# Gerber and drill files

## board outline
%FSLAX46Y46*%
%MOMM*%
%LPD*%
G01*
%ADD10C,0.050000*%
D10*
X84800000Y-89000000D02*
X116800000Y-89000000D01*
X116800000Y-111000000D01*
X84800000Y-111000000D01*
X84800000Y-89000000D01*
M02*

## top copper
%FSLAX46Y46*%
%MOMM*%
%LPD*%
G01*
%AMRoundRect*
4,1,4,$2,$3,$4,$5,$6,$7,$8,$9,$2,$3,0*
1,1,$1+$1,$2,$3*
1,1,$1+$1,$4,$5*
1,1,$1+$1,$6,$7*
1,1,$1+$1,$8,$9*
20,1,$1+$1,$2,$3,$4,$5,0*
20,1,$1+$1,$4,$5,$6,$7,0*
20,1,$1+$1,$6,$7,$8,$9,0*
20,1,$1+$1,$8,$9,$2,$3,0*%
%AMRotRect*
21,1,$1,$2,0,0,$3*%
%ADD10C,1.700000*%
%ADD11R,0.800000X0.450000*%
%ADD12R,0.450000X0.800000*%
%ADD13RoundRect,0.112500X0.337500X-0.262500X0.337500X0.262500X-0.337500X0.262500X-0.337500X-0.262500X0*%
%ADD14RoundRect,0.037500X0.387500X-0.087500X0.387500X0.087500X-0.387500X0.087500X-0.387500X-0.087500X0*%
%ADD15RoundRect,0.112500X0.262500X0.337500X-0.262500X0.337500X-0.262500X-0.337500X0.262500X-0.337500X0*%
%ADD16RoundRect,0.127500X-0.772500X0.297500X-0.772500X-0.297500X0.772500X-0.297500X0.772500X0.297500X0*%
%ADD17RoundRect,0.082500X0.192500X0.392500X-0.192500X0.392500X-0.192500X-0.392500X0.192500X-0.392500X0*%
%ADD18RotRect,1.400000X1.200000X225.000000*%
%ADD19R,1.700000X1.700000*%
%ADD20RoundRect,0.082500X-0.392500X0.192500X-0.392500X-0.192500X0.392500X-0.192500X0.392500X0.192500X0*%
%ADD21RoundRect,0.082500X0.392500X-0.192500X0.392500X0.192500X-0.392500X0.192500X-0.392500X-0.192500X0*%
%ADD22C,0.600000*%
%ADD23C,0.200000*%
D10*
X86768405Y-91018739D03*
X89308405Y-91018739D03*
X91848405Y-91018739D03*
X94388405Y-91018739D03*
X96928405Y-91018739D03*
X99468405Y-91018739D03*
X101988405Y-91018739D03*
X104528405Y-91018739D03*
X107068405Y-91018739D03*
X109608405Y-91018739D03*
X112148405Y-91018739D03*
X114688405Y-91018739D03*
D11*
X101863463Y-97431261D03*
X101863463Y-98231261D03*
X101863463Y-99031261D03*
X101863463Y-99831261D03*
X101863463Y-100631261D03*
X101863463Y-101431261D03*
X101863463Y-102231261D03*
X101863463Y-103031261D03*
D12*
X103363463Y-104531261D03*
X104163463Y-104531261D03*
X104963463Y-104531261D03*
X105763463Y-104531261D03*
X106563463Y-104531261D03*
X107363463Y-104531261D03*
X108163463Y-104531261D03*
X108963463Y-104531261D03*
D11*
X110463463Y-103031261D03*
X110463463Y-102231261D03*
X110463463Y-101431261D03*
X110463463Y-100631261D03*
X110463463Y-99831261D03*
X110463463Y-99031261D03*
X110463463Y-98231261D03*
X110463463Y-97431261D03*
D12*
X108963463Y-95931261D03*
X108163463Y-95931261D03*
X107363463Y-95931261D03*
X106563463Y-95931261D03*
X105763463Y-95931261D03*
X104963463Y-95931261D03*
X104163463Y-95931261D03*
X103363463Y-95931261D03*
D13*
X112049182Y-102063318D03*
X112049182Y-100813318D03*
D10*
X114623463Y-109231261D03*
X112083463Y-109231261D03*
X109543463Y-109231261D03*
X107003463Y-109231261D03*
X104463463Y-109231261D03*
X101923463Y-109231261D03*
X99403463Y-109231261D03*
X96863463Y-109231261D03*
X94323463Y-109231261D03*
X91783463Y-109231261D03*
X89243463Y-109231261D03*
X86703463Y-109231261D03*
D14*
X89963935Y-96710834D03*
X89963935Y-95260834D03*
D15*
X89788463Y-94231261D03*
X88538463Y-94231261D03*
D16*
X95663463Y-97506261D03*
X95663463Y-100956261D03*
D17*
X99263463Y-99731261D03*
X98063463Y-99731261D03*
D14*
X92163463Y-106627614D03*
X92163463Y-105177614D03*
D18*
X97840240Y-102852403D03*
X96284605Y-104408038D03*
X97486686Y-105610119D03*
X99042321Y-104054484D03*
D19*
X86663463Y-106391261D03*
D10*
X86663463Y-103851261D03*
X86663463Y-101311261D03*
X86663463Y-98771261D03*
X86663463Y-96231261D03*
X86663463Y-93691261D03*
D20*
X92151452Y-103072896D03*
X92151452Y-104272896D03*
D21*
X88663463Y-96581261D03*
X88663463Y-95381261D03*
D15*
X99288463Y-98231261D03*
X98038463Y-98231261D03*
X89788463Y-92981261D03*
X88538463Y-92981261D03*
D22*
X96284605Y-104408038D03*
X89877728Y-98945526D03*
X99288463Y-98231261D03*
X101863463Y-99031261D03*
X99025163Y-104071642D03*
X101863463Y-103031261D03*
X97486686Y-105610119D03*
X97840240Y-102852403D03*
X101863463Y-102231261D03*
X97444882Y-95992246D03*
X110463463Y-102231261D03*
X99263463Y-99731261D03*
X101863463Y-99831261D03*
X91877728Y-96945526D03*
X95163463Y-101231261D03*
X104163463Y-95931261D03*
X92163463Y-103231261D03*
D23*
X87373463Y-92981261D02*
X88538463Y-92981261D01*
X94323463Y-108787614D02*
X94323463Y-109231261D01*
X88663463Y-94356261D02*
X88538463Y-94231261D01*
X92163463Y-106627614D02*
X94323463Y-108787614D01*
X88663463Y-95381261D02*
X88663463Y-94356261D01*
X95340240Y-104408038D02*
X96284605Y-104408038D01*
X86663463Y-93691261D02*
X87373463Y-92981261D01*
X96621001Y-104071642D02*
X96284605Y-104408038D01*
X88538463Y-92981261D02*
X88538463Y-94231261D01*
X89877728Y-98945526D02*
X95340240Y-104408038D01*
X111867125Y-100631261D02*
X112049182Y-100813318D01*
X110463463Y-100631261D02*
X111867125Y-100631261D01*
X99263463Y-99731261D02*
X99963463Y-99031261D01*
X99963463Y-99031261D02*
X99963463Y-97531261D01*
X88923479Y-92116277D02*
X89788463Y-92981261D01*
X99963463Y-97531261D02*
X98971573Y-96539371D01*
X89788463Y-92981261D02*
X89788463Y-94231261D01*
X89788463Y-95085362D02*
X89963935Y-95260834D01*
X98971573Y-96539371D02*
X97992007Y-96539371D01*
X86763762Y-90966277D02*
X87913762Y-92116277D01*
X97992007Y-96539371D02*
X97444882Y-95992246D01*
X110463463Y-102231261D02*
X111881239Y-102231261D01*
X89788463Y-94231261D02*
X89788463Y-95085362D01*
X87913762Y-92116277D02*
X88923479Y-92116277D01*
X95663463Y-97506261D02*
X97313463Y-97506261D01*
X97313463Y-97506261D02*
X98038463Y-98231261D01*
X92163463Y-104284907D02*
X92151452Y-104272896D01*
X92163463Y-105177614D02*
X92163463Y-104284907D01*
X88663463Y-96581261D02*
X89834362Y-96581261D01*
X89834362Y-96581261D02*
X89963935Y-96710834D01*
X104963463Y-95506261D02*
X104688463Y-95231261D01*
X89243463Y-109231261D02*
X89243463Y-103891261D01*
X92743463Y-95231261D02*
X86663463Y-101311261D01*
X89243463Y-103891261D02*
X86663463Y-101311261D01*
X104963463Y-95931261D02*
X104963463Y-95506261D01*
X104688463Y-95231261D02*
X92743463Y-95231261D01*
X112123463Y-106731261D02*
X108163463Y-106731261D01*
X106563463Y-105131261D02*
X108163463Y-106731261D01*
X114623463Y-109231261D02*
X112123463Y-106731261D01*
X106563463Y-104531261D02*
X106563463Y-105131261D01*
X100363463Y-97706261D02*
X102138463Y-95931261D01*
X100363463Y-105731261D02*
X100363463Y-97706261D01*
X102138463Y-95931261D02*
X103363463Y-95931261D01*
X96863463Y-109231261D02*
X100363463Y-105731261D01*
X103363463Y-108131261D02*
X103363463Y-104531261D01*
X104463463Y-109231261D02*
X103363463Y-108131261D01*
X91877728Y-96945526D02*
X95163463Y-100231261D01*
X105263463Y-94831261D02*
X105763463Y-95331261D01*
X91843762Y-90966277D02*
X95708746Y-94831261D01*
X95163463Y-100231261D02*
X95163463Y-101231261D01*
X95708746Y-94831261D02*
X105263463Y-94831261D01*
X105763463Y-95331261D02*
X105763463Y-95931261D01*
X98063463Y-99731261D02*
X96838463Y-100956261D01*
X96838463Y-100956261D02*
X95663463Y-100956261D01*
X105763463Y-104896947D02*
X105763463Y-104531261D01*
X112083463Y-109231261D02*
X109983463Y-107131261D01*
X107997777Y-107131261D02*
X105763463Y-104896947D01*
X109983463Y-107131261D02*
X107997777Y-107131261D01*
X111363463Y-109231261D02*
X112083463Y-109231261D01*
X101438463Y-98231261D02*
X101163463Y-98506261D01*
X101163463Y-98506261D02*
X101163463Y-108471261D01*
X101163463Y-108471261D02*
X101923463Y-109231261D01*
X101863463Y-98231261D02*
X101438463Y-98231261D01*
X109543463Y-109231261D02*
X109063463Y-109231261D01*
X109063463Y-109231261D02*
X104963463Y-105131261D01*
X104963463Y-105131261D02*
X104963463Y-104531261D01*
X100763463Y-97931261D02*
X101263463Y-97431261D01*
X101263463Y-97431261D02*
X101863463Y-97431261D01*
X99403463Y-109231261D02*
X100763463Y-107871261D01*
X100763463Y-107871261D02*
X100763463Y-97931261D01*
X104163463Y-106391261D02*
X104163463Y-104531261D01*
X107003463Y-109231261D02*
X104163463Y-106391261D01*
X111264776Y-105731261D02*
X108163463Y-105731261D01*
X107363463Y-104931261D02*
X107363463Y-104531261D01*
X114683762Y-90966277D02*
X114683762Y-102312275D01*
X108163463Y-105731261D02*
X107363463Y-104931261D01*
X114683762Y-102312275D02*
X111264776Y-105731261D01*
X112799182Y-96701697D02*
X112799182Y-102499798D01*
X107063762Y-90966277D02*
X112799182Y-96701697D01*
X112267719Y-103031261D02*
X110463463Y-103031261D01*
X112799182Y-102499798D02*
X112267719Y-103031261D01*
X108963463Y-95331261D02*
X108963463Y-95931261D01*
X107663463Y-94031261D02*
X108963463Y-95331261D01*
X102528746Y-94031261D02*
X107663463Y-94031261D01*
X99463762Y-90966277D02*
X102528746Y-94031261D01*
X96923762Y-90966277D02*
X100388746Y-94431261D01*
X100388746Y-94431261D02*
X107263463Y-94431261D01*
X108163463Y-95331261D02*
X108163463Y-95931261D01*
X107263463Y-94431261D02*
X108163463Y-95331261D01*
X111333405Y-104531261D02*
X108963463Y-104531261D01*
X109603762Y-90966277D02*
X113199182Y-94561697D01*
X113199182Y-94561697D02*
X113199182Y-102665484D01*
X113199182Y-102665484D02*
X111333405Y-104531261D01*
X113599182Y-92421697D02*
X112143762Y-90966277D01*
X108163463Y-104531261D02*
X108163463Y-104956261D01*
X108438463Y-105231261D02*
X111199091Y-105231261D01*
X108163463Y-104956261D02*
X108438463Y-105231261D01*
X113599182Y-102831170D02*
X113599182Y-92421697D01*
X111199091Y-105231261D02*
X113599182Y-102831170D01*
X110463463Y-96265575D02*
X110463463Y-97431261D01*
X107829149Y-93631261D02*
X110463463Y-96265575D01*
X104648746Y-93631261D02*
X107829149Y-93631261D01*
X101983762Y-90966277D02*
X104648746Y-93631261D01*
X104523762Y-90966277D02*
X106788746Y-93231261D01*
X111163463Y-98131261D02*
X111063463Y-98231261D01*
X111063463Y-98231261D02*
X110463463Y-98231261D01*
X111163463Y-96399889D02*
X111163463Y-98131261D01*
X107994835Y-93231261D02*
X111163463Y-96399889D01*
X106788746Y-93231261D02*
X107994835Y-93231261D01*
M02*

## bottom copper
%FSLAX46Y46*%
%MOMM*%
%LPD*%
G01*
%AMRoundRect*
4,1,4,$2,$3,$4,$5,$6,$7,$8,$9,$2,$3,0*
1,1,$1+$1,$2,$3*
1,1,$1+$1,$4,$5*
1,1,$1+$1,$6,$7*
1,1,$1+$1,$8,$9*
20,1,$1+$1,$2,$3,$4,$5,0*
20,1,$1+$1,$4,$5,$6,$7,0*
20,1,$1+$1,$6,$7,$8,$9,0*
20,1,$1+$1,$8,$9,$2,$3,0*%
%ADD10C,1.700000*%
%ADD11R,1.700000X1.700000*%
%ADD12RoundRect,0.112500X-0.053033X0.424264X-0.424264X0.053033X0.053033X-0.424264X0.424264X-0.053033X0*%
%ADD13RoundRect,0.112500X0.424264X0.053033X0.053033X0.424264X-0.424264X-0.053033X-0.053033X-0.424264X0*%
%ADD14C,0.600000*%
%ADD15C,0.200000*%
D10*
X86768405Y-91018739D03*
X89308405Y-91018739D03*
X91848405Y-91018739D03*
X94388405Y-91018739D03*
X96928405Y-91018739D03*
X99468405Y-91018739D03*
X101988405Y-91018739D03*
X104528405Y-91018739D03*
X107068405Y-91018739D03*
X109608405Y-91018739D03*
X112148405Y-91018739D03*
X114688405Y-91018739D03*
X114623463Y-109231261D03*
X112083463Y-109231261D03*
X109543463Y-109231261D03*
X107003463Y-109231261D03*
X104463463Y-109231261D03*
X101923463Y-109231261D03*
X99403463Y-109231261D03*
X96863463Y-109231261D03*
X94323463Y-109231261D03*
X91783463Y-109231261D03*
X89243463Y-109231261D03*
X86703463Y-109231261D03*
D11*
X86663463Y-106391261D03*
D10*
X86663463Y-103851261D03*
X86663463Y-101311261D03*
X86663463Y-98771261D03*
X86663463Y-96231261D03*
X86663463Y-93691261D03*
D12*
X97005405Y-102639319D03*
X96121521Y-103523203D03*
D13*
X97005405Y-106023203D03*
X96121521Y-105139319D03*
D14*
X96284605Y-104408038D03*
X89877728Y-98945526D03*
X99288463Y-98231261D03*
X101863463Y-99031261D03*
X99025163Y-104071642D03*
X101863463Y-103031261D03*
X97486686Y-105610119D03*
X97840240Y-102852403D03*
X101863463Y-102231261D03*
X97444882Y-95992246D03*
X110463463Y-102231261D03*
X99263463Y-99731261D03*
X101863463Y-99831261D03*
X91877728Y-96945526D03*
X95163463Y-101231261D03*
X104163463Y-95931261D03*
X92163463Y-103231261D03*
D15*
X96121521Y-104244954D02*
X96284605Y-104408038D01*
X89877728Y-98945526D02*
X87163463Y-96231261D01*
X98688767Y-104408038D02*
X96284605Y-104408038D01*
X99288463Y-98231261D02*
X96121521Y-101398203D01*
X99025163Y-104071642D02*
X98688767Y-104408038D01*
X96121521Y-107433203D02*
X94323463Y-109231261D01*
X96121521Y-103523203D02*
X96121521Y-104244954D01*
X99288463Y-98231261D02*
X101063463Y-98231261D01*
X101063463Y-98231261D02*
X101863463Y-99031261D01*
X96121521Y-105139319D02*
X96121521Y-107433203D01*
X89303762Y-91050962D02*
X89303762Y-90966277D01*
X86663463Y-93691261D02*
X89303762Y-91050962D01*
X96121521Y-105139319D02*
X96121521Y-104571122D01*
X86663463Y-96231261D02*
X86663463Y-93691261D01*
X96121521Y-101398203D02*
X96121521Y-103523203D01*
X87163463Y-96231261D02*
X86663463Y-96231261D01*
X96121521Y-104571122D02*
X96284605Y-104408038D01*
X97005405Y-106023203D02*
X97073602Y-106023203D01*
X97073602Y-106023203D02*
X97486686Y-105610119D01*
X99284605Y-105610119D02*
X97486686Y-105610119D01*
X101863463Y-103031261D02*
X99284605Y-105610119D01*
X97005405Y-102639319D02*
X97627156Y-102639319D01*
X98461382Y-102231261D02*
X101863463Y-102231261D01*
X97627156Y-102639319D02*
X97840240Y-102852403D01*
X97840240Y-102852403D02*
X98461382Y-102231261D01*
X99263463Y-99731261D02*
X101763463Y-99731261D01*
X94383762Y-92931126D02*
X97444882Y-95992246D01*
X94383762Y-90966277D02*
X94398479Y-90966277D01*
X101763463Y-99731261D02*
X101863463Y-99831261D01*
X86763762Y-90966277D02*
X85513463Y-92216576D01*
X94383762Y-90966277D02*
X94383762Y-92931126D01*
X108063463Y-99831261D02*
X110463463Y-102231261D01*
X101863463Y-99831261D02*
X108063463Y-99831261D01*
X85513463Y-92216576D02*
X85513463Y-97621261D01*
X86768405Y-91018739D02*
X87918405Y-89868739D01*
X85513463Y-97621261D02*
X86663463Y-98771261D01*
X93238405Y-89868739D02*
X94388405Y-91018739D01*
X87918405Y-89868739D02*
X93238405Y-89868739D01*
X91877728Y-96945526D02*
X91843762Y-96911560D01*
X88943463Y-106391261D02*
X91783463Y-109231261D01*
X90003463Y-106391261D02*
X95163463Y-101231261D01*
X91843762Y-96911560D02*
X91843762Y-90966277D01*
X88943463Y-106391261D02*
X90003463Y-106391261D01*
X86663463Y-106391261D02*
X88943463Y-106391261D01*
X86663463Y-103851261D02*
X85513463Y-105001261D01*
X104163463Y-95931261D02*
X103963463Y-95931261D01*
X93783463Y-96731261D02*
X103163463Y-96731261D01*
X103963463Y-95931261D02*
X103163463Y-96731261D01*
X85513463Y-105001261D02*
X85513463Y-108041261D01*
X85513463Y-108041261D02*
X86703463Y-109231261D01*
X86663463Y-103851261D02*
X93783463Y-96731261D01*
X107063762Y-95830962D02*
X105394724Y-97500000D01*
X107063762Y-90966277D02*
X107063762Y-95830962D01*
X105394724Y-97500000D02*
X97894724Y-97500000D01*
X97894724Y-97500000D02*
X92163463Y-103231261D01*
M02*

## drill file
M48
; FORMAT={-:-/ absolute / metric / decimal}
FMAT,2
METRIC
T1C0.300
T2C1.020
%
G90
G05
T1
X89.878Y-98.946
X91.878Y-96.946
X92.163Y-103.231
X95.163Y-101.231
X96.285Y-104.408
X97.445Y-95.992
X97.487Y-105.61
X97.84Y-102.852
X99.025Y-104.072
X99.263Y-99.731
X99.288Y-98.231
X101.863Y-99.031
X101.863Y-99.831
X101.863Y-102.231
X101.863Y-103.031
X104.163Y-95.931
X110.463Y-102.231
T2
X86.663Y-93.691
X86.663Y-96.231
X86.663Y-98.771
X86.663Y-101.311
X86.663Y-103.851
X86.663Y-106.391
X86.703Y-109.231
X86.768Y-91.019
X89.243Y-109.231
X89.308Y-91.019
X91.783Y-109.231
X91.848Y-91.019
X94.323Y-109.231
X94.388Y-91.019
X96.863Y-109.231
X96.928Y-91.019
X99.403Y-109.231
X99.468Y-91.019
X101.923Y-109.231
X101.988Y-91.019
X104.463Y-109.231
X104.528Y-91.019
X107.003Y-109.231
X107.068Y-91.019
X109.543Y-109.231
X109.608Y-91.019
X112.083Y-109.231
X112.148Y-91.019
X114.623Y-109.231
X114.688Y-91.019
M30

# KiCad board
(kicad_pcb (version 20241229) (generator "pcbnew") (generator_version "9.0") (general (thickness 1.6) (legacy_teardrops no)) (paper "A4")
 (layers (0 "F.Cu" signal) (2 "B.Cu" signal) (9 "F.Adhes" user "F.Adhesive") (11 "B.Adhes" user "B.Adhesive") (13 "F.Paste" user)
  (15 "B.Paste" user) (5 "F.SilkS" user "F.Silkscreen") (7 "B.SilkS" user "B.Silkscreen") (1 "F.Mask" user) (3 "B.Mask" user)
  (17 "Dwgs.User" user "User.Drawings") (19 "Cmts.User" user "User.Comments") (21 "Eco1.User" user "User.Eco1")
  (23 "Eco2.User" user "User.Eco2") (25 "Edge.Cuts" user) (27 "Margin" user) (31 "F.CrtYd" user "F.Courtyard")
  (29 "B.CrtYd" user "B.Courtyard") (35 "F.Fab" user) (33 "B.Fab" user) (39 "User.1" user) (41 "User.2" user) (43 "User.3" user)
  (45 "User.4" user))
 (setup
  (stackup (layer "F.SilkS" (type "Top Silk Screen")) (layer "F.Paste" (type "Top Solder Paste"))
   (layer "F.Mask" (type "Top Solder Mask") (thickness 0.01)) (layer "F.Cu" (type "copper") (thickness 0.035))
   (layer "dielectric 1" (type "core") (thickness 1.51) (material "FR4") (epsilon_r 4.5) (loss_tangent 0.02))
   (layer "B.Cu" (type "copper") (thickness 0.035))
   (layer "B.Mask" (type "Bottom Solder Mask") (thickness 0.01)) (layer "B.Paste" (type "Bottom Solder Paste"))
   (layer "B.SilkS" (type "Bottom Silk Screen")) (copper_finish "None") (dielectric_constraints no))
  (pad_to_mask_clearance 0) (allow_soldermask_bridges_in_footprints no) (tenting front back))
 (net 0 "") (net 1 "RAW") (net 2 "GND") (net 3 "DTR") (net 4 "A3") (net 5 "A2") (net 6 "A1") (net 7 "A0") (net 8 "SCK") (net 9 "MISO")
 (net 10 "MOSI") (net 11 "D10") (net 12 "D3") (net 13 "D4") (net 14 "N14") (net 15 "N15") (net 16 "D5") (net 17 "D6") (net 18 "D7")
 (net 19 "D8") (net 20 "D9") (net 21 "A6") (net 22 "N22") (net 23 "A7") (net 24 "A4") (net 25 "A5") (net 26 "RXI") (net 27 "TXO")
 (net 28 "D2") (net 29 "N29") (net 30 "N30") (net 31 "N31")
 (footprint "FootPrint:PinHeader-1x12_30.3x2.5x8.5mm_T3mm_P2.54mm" (layer "F.Cu") (at 100.728405 91.018739)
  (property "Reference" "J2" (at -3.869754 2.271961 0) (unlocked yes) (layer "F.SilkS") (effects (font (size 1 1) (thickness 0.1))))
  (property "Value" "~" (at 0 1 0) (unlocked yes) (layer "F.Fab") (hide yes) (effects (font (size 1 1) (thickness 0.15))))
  (pad "1" thru_hole circle (at -13.96 0) (size 1.7 1.7) (drill 1.02) (layers "*.Cu" "*.Mask") (remove_unused_layers no) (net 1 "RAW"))
  (pad "2" thru_hole circle (at -11.42 0) (size 1.7 1.7) (drill 1.02) (layers "*.Cu" "*.Mask") (remove_unused_layers no) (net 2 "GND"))
  (pad "3" thru_hole circle (at -8.88 0) (size 1.7 1.7) (drill 1.02) (layers "*.Cu" "*.Mask") (remove_unused_layers no) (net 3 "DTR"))
  (pad "4" thru_hole circle (at -6.34 0) (size 1.7 1.7) (drill 1.02) (layers "*.Cu" "*.Mask") (remove_unused_layers no) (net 1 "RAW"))
  (pad "5" thru_hole circle (at -3.8 0) (size 1.7 1.7) (drill 1.02) (layers "*.Cu" "*.Mask") (remove_unused_layers no) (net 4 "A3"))
  (pad "6" thru_hole circle (at -1.26 0) (size 1.7 1.7) (drill 1.02) (layers "*.Cu" "*.Mask") (remove_unused_layers no) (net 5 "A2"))
  (pad "7" thru_hole circle (at 1.26 0) (size 1.7 1.7) (drill 1.02) (layers "*.Cu" "*.Mask") (remove_unused_layers no) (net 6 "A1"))
  (pad "8" thru_hole circle (at 3.8 0) (size 1.7 1.7) (drill 1.02) (layers "*.Cu" "*.Mask") (remove_unused_layers no) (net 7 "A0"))
  (pad "9" thru_hole circle (at 6.34 0) (size 1.7 1.7) (drill 1.02) (layers "*.Cu" "*.Mask") (remove_unused_layers no) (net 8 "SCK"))
  (pad "10" thru_hole circle (at 8.88 0) (size 1.7 1.7) (drill 1.02) (layers "*.Cu" "*.Mask") (remove_unused_layers no) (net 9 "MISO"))
  (pad "11" thru_hole circle (at 11.42 0) (size 1.7 1.7) (drill 1.02) (layers "*.Cu" "*.Mask") (remove_unused_layers no) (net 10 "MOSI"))
  (pad "12" thru_hole circle (at 13.96 0) (size 1.7 1.7) (drill 1.02) (layers "*.Cu" "*.Mask") (remove_unused_layers no) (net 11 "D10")))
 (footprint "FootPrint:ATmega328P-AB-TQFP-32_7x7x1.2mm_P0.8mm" (layer "F.Cu") (at 106.163463 100.231261)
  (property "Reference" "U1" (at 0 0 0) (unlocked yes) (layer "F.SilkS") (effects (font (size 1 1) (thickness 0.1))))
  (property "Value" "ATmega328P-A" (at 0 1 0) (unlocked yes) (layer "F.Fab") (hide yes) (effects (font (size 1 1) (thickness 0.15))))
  (pad "1" smd rect (at -4.3 -2.8) (size 0.8 0.45) (layers "F.Cu" "F.Mask" "F.Paste") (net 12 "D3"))
  (pad "2" smd rect (at -4.3 -2) (size 0.8 0.45) (layers "F.Cu" "F.Mask" "F.Paste") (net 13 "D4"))
  (pad "3" smd rect (at -4.3 -1.2) (size 0.8 0.45) (layers "F.Cu" "F.Mask" "F.Paste") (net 2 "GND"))
  (pad "4" smd rect (at -4.3 -0.4) (size 0.8 0.45) (layers "F.Cu" "F.Mask" "F.Paste") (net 1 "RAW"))
  (pad "5" smd rect (at -4.3 0.4) (size 0.8 0.45) (layers "F.Cu" "F.Mask" "F.Paste"))
  (pad "6" smd rect (at -4.3 1.2) (size 0.8 0.45) (layers "F.Cu" "F.Mask" "F.Paste"))
  (pad "7" smd rect (at -4.3 2) (size 0.8 0.45) (layers "F.Cu" "F.Mask" "F.Paste") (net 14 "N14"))
  (pad "8" smd rect (at -4.3 2.8) (size 0.8 0.45) (layers "F.Cu" "F.Mask" "F.Paste") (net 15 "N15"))
  (pad "9" smd rect (at -2.8 4.3 90) (size 0.8 0.45) (layers "F.Cu" "F.Mask" "F.Paste") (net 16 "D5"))
  (pad "10" smd rect (at -2 4.3 90) (size 0.8 0.45) (layers "F.Cu" "F.Mask" "F.Paste") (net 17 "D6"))
  (pad "11" smd rect (at -1.2 4.3 90) (size 0.8 0.45) (layers "F.Cu" "F.Mask" "F.Paste") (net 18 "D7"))
  (pad "12" smd rect (at -0.4 4.3 90) (size 0.8 0.45) (layers "F.Cu" "F.Mask" "F.Paste") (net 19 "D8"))
  (pad "13" smd rect (at 0.4 4.3 90) (size 0.8 0.45) (layers "F.Cu" "F.Mask" "F.Paste") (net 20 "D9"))
  (pad "14" smd rect (at 1.2 4.3 90) (size 0.8 0.45) (layers "F.Cu" "F.Mask" "F.Paste") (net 11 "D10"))
  (pad "15" smd rect (at 2 4.3 90) (size 0.8 0.45) (layers "F.Cu" "F.Mask" "F.Paste") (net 10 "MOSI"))
  (pad "16" smd rect (at 2.8 4.3 90) (size 0.8 0.45) (layers "F.Cu" "F.Mask" "F.Paste") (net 9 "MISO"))
  (pad "17" smd rect (at 4.3 2.8) (size 0.8 0.45) (layers "F.Cu" "F.Mask" "F.Paste") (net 8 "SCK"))
  (pad "18" smd rect (at 4.3 2) (size 0.8 0.45) (layers "F.Cu" "F.Mask" "F.Paste") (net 1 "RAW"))
  (pad "19" smd rect (at 4.3 1.2) (size 0.8 0.45) (layers "F.Cu" "F.Mask" "F.Paste") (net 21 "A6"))
  (pad "20" smd rect (at 4.3 0.4) (size 0.8 0.45) (layers "F.Cu" "F.Mask" "F.Paste") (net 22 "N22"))
  (pad "21" smd rect (at 4.3 -0.4) (size 0.8 0.45) (layers "F.Cu" "F.Mask" "F.Paste"))
  (pad "22" smd rect (at 4.3 -1.2) (size 0.8 0.45) (layers "F.Cu" "F.Mask" "F.Paste") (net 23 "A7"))
  (pad "23" smd rect (at 4.3 -2) (size 0.8 0.45) (layers "F.Cu" "F.Mask" "F.Paste") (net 7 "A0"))
  (pad "24" smd rect (at 4.3 -2.8) (size 0.8 0.45) (layers "F.Cu" "F.Mask" "F.Paste") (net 6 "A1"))
  (pad "25" smd rect (at 2.8 -4.3 90) (size 0.8 0.45) (layers "F.Cu" "F.Mask" "F.Paste") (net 5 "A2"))
  (pad "26" smd rect (at 2 -4.3 90) (size 0.8 0.45) (layers "F.Cu" "F.Mask" "F.Paste") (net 4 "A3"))
  (pad "27" smd rect (at 1.2 -4.3 90) (size 0.8 0.45) (layers "F.Cu" "F.Mask" "F.Paste") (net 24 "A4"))
  (pad "28" smd rect (at 0.4 -4.3 90) (size 0.8 0.45) (layers "F.Cu" "F.Mask" "F.Paste") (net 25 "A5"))
  (pad "29" smd rect (at -0.4 -4.3 90) (size 0.8 0.45) (layers "F.Cu" "F.Mask" "F.Paste") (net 3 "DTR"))
  (pad "30" smd rect (at -1.2 -4.3 90) (size 0.8 0.45) (layers "F.Cu" "F.Mask" "F.Paste") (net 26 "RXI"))
  (pad "31" smd rect (at -2 -4.3 90) (size 0.8 0.45) (layers "F.Cu" "F.Mask" "F.Paste") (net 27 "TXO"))
  (pad "32" smd rect (at -2.8 -4.3 90) (size 0.8 0.45) (layers "F.Cu" "F.Mask" "F.Paste") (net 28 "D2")))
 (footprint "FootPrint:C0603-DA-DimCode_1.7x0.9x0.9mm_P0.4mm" (layer "F.Cu") (at 112.049182 101.438318 90)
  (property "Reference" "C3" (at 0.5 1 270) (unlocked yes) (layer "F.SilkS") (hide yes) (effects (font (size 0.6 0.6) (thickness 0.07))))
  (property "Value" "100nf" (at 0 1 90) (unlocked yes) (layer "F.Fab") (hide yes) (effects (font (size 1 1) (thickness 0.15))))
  (pad "1" smd roundrect (at -0.625 0 90) (size 0.75 0.9) (layers "F.Cu" "F.Mask" "F.Paste") (roundrect_rratio 0.15) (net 1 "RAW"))
  (pad "2" smd roundrect (at 0.625 0 90) (size 0.75 0.9) (layers "F.Cu" "F.Mask" "F.Paste") (roundrect_rratio 0.15) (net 22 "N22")))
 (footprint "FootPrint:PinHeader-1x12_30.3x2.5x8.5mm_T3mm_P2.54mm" (layer "F.Cu") (at 100.663463 109.231261 180)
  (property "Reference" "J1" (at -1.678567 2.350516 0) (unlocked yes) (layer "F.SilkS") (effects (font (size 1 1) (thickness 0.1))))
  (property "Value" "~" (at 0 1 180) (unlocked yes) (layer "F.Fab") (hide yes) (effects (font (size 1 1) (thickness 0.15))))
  (pad "1" thru_hole circle (at -13.96 0 180) (size 1.7 1.7) (drill 1.02) (layers "*.Cu" "*.Mask") (remove_unused_layers no) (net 20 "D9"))
  (pad "2" thru_hole circle (at -11.42 0 180) (size 1.7 1.7) (drill 1.02) (layers "*.Cu" "*.Mask") (remove_unused_layers no) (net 19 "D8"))
  (pad "3" thru_hole circle (at -8.88 0 180) (size 1.7 1.7) (drill 1.02) (layers "*.Cu" "*.Mask") (remove_unused_layers no) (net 18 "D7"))
  (pad "4" thru_hole circle (at -6.34 0 180) (size 1.7 1.7) (drill 1.02) (layers "*.Cu" "*.Mask") (remove_unused_layers no) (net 17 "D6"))
  (pad "5" thru_hole circle (at -3.8 0 180) (size 1.7 1.7) (drill 1.02) (layers "*.Cu" "*.Mask") (remove_unused_layers no) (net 16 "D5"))
  (pad "6" thru_hole circle (at -1.26 0 180) (size 1.7 1.7) (drill 1.02) (layers "*.Cu" "*.Mask") (remove_unused_layers no) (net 13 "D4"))
  (pad "7" thru_hole circle (at 1.26 0 180) (size 1.7 1.7) (drill 1.02) (layers "*.Cu" "*.Mask") (remove_unused_layers no) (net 12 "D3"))
  (pad "8" thru_hole circle (at 3.8 0 180) (size 1.7 1.7) (drill 1.02) (layers "*.Cu" "*.Mask") (remove_unused_layers no) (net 28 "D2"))
  (pad "9" thru_hole circle (at 6.34 0 180) (size 1.7 1.7) (drill 1.02) (layers "*.Cu" "*.Mask") (remove_unused_layers no) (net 2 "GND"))
  (pad "10" thru_hole circle (at 8.88 0 180) (size 1.7 1.7) (drill 1.02) (layers "*.Cu" "*.Mask") (remove_unused_layers no) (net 3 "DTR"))
  (pad "11" thru_hole circle (at 11.42 0 180) (size 1.7 1.7) (drill 1.02) (layers "*.Cu" "*.Mask") (remove_unused_layers no) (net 26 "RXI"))
  (pad "12" thru_hole circle (at 13.96 0 180) (size 1.7 1.7) (drill 1.02) (layers "*.Cu" "*.Mask") (remove_unused_layers no) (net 27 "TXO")))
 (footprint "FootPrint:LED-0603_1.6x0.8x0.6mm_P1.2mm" (layer "F.Cu") (at 89.963935 95.985834 90)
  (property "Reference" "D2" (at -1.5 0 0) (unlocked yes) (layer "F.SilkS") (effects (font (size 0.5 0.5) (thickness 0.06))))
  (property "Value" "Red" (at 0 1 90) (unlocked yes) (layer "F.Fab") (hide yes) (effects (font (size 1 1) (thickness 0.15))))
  (pad "1" smd roundrect (at -0.725 0 90) (size 0.25 0.85) (layers "F.Cu" "F.Mask" "F.Paste") (roundrect_rratio 0.15) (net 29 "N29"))
  (pad "2" smd roundrect (at 0.725 0 90) (size 0.25 0.85) (layers "F.Cu" "F.Mask" "F.Paste") (roundrect_rratio 0.15) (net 1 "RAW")))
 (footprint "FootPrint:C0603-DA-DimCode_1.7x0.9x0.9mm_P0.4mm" (layer "F.Cu") (at 89.163463 94.231261 180)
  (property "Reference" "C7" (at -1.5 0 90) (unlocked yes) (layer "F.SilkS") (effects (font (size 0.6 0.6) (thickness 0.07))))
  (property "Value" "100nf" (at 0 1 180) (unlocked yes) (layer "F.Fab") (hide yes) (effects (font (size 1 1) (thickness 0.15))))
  (pad "1" smd roundrect (at -0.625 0 180) (size 0.75 0.9) (layers "F.Cu" "F.Mask" "F.Paste") (roundrect_rratio 0.15) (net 1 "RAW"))
  (pad "2" smd roundrect (at 0.625 0 180) (size 0.75 0.9) (layers "F.Cu" "F.Mask" "F.Paste") (roundrect_rratio 0.15) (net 2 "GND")))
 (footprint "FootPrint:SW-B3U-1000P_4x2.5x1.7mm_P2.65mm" (layer "F.Cu") (at 95.663463 99.231261 -90)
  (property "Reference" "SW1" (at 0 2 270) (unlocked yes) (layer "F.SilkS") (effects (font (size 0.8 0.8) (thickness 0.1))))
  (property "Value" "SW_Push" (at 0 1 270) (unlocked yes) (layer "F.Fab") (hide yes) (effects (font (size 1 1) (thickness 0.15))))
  (pad "1" smd roundrect (at -1.725 0 270) (size 0.85 1.8) (layers "F.Cu" "F.Mask" "F.Paste") (roundrect_rratio 0.15) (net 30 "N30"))
  (pad "2" smd roundrect (at 1.725 0 270) (size 0.85 1.8) (layers "F.Cu" "F.Mask" "F.Paste") (roundrect_rratio 0.15) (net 3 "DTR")))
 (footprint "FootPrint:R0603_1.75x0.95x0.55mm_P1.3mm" (layer "F.Cu") (at 98.663463 99.731261 180)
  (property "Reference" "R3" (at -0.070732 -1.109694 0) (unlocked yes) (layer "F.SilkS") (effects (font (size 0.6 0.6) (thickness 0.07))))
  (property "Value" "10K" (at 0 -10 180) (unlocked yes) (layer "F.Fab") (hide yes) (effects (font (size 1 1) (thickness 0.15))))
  (pad "1" smd roundrect (at -0.6 0 180) (size 0.55 0.95) (layers "F.Cu" "F.Mask" "F.Paste") (roundrect_rratio 0.15) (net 1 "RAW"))
  (pad "2" smd roundrect (at 0.6 0 180) (size 0.55 0.95) (layers "F.Cu" "F.Mask" "F.Paste") (roundrect_rratio 0.15) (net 3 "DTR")))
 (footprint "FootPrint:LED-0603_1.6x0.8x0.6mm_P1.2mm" (layer "F.Cu") (at 92.163463 105.902614 90)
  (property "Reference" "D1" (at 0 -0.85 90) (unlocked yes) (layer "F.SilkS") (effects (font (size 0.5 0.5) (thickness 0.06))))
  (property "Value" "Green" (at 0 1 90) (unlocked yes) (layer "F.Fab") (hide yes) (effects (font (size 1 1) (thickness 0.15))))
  (pad "1" smd roundrect (at -0.725 0 90) (size 0.25 0.85) (layers "F.Cu" "F.Mask" "F.Paste") (roundrect_rratio 0.15) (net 2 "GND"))
  (pad "2" smd roundrect (at 0.725 0 90) (size 0.25 0.85) (layers "F.Cu" "F.Mask" "F.Paste") (roundrect_rratio 0.15) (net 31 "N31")))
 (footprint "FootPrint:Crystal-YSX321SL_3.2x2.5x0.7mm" (layer "F.Cu") (at 97.663463 104.231261 -135)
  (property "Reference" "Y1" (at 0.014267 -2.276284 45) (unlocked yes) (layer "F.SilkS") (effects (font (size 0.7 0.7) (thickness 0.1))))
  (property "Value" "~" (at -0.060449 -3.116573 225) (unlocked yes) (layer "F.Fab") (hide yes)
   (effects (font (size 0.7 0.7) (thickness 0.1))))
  (pad "1" smd rect (at -1.1 0.85 225) (size 1.4 1.2) (layers "F.Cu" "F.Mask" "F.Paste") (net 14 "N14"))
  (pad "2" smd rect (at 1.1 0.85 225) (size 1.4 1.2) (layers "F.Cu" "F.Mask" "F.Paste") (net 2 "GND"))
  (pad "3" smd rect (at 1.1 -0.85 225) (size 1.4 1.2) (layers "F.Cu" "F.Mask" "F.Paste") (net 15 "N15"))
  (pad "4" smd rect (at -1.1 -0.85 225) (size 1.4 1.2) (layers "F.Cu" "F.Mask" "F.Paste") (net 2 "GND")))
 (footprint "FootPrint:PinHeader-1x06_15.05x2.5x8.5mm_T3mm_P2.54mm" (layer "F.Cu") (at 86.663463 100.041261 90)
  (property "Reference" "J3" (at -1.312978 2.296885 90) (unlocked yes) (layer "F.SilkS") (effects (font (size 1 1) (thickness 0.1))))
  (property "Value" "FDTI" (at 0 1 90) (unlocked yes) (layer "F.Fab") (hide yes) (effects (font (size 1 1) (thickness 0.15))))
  (pad "1" thru_hole rect (at -6.35 0 90) (size 1.7 1.7) (drill 1.02) (layers "*.Cu" "*.Mask") (remove_unused_layers no) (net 3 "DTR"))
  (pad "2" thru_hole circle (at -3.81 0 90) (size 1.7 1.7) (drill 1.02) (layers "*.Cu" "*.Mask") (remove_unused_layers no) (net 27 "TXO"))
  (pad "3" thru_hole circle (at -1.27 0 90) (size 1.7 1.7) (drill 1.02) (layers "*.Cu" "*.Mask") (remove_unused_layers no) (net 26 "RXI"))
  (pad "4" thru_hole circle (at 1.27 0 90) (size 1.7 1.7) (drill 1.02) (layers "*.Cu" "*.Mask") (remove_unused_layers no) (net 1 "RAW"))
  (pad "5" thru_hole circle (at 3.81 0 90) (size 1.7 1.7) (drill 1.02) (layers "*.Cu" "*.Mask") (remove_unused_layers no) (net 2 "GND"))
  (pad "6" thru_hole circle (at 6.35 0 90) (size 1.7 1.7) (drill 1.02) (layers "*.Cu" "*.Mask") (remove_unused_layers no) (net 2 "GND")))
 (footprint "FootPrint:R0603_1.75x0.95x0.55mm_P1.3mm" (layer "F.Cu") (at 92.151452 103.672896 -90)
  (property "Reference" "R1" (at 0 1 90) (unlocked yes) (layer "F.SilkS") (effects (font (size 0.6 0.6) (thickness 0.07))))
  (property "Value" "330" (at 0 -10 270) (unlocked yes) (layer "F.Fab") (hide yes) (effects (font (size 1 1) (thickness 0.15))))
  (pad "1" smd roundrect (at -0.6 0 270) (size 0.55 0.95) (layers "F.Cu" "F.Mask" "F.Paste") (roundrect_rratio 0.15) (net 8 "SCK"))
  (pad "2" smd roundrect (at 0.6 0 270) (size 0.55 0.95) (layers "F.Cu" "F.Mask" "F.Paste") (roundrect_rratio 0.15) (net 31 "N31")))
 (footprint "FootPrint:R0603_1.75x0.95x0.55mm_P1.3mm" (layer "F.Cu") (at 88.663463 95.981261 90)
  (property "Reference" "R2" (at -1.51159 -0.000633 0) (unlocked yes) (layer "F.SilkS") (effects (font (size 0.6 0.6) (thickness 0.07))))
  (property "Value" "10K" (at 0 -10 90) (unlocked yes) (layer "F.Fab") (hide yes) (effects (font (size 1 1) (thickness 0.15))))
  (pad "1" smd roundrect (at -0.6 0 90) (size 0.55 0.95) (layers "F.Cu" "F.Mask" "F.Paste") (roundrect_rratio 0.15) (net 29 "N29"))
  (pad "2" smd roundrect (at 0.6 0 90) (size 0.55 0.95) (layers "F.Cu" "F.Mask" "F.Paste") (roundrect_rratio 0.15) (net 2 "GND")))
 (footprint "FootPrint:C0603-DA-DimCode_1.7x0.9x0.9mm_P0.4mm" (layer "F.Cu") (at 98.663463 98.231261 180)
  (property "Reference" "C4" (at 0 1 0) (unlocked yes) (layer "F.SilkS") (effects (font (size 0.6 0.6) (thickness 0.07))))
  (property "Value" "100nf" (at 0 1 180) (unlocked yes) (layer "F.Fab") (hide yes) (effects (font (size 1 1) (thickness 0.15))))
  (pad "1" smd roundrect (at -0.625 0 180) (size 0.75 0.9) (layers "F.Cu" "F.Mask" "F.Paste") (roundrect_rratio 0.15) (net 2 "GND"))
  (pad "2" smd roundrect (at 0.625 0 180) (size 0.75 0.9) (layers "F.Cu" "F.Mask" "F.Paste") (roundrect_rratio 0.15) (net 30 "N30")))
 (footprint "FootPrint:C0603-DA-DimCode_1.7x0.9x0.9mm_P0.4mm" (layer "F.Cu") (at 89.163463 92.981261 180)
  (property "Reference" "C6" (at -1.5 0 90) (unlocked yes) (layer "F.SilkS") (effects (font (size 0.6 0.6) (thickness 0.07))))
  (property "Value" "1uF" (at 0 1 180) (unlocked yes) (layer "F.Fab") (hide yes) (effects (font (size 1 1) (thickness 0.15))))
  (pad "1" smd roundrect (at -0.625 0 180) (size 0.75 0.9) (layers "F.Cu" "F.Mask" "F.Paste") (roundrect_rratio 0.15) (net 1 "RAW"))
  (pad "2" smd roundrect (at 0.625 0 180) (size 0.75 0.9) (layers "F.Cu" "F.Mask" "F.Paste") (roundrect_rratio 0.15) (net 2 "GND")))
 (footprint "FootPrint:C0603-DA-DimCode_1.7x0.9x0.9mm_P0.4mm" (layer "B.Cu") (at 96.563463 103.081261 -135)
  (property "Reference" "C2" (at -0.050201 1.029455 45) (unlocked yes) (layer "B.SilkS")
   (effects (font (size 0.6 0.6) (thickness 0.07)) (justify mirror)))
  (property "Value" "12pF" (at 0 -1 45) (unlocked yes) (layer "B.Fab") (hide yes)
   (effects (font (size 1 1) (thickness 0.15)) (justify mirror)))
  (pad "1" smd roundrect (at -0.625 0 225) (size 0.75 0.9) (layers "B.Cu" "B.Mask" "B.Paste") (roundrect_rratio 0.15) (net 14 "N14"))
  (pad "2" smd roundrect (at 0.625 0 225) (size 0.75 0.9) (layers "B.Cu" "B.Mask" "B.Paste") (roundrect_rratio 0.15) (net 2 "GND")))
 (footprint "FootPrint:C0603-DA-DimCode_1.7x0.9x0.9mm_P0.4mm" (layer "B.Cu") (at 96.563463 105.581261 135)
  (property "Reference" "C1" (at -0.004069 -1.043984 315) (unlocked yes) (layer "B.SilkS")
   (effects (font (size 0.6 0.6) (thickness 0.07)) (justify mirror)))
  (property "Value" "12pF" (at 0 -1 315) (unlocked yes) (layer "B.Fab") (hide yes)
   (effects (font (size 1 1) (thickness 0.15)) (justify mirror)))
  (pad "1" smd roundrect (at -0.625 0 135) (size 0.75 0.9) (layers "B.Cu" "B.Mask" "B.Paste") (roundrect_rratio 0.15) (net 15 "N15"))
  (pad "2" smd roundrect (at 0.625 0 135) (size 0.75 0.9) (layers "B.Cu" "B.Mask" "B.Paste") (roundrect_rratio 0.15) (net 2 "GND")))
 (gr_rect (start 84.8 89) (end 116.8 111) (stroke (width 0.05) (type solid)) (fill no) (layer "Edge.Cuts"))
 (segment (start 87.373463 92.981261) (end 88.538463 92.981261) (width 0.2) (layer "F.Cu") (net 2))
 (segment (start 94.323463 108.787614) (end 94.323463 109.231261) (width 0.2) (layer "F.Cu") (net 2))
 (segment (start 88.663463 94.356261) (end 88.538463 94.231261) (width 0.2) (layer "F.Cu") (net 2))
 (segment (start 92.163463 106.627614) (end 94.323463 108.787614) (width 0.2) (layer "F.Cu") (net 2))
 (segment (start 88.663463 95.381261) (end 88.663463 94.356261) (width 0.2) (layer "F.Cu") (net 2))
 (segment (start 95.34024 104.408038) (end 96.284605 104.408038) (width 0.2) (layer "F.Cu") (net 2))
 (segment (start 86.663463 93.691261) (end 87.373463 92.981261) (width 0.2) (layer "F.Cu") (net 2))
 (segment (start 96.621001 104.071642) (end 96.284605 104.408038) (width 0.2) (layer "F.Cu") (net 2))
 (segment (start 88.538463 92.981261) (end 88.538463 94.231261) (width 0.2) (layer "F.Cu") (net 2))
 (segment (start 89.877728 98.945526) (end 95.34024 104.408038) (width 0.2) (layer "F.Cu") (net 2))
 (via (at 96.284605 104.408038) (size 0.6) (drill 0.3) (layers "F.Cu" "B.Cu") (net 2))
 (via (at 89.877728 98.945526) (size 0.6) (drill 0.3) (layers "F.Cu" "B.Cu") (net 2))
 (via (at 99.288463 98.231261) (size 0.6) (drill 0.3) (layers "F.Cu" "B.Cu") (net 2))
 (via (at 101.863463 99.031261) (size 0.6) (drill 0.3) (layers "F.Cu" "B.Cu") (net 2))
 (via (at 99.025163 104.071642) (size 0.6) (drill 0.3) (layers "F.Cu" "B.Cu") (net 2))
 (segment (start 96.121521 104.244954) (end 96.284605 104.408038) (width 0.2) (layer "B.Cu") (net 2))
 (segment (start 89.877728 98.945526) (end 87.163463 96.231261) (width 0.2) (layer "B.Cu") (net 2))
 (segment (start 98.688767 104.408038) (end 96.284605 104.408038) (width 0.2) (layer "B.Cu") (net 2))
 (segment (start 99.288463 98.231261) (end 96.121521 101.398203) (width 0.2) (layer "B.Cu") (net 2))
 (segment (start 99.025163 104.071642) (end 98.688767 104.408038) (width 0.2) (layer "B.Cu") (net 2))
 (segment (start 96.121521 107.433203) (end 94.323463 109.231261) (width 0.2) (layer "B.Cu") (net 2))
 (segment (start 96.121521 103.523203) (end 96.121521 104.244954) (width 0.2) (layer "B.Cu") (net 2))
 (segment (start 99.288463 98.231261) (end 101.063463 98.231261) (width 0.2) (layer "B.Cu") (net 2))
 (segment (start 101.063463 98.231261) (end 101.863463 99.031261) (width 0.2) (layer "B.Cu") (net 2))
 (segment (start 96.121521 105.139319) (end 96.121521 107.433203) (width 0.2) (layer "B.Cu") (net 2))
 (segment (start 89.303762 91.050962) (end 89.303762 90.966277) (width 0.2) (layer "B.Cu") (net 2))
 (segment (start 86.663463 93.691261) (end 89.303762 91.050962) (width 0.2) (layer "B.Cu") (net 2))
 (segment (start 96.121521 105.139319) (end 96.121521 104.571122) (width 0.2) (layer "B.Cu") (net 2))
 (segment (start 86.663463 96.231261) (end 86.663463 93.691261) (width 0.2) (layer "B.Cu") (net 2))
 (segment (start 96.121521 101.398203) (end 96.121521 103.523203) (width 0.2) (layer "B.Cu") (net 2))
 (segment (start 87.163463 96.231261) (end 86.663463 96.231261) (width 0.2) (layer "B.Cu") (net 2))
 (segment (start 96.121521 104.571122) (end 96.284605 104.408038) (width 0.2) (layer "B.Cu") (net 2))
 (via (at 101.863463 103.031261) (size 0.6) (drill 0.3) (layers "F.Cu" "B.Cu") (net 15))
 (via (at 97.486686 105.610119) (size 0.6) (drill 0.3) (layers "F.Cu" "B.Cu") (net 15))
 (segment (start 97.005405 106.023203) (end 97.073602 106.023203) (width 0.2) (layer "B.Cu") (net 15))
 (segment (start 97.073602 106.023203) (end 97.486686 105.610119) (width 0.2) (layer "B.Cu") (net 15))
 (segment (start 99.284605 105.610119) (end 97.486686 105.610119) (width 0.2) (layer "B.Cu") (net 15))
 (segment (start 101.863463 103.031261) (end 99.284605 105.610119) (width 0.2) (layer "B.Cu") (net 15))
 (via (at 97.84024 102.852403) (size 0.6) (drill 0.3) (layers "F.Cu" "B.Cu") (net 14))
 (via (at 101.863463 102.231261) (size 0.6) (drill 0.3) (layers "F.Cu" "B.Cu") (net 14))
 (segment (start 97.005405 102.639319) (end 97.627156 102.639319) (width 0.2) (layer "B.Cu") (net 14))
 (segment (start 98.461382 102.231261) (end 101.863463 102.231261) (width 0.2) (layer "B.Cu") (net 14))
 (segment (start 97.627156 102.639319) (end 97.84024 102.852403) (width 0.2) (layer "B.Cu") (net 14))
 (segment (start 97.84024 102.852403) (end 98.461382 102.231261) (width 0.2) (layer "B.Cu") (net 14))
 (segment (start 111.867125 100.631261) (end 112.049182 100.813318) (width 0.2) (layer "F.Cu") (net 22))
 (segment (start 110.463463 100.631261) (end 111.867125 100.631261) (width 0.2) (layer "F.Cu") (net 22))
 (segment (start 99.263463 99.731261) (end 99.963463 99.031261) (width 0.2) (layer "F.Cu") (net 1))
 (segment (start 99.963463 99.031261) (end 99.963463 97.531261) (width 0.2) (layer "F.Cu") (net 1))
 (segment (start 88.923479 92.116277) (end 89.788463 92.981261) (width 0.2) (layer "F.Cu") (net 1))
 (segment (start 99.963463 97.531261) (end 98.971573 96.539371) (width 0.2) (layer "F.Cu") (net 1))
 (segment (start 89.788463 92.981261) (end 89.788463 94.231261) (width 0.2) (layer "F.Cu") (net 1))
 (segment (start 89.788463 95.085362) (end 89.963935 95.260834) (width 0.2) (layer "F.Cu") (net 1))
 (segment (start 98.971573 96.539371) (end 97.992007 96.539371) (width 0.2) (layer "F.Cu") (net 1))
 (segment (start 86.763762 90.966277) (end 87.913762 92.116277) (width 0.2) (layer "F.Cu") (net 1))
 (segment (start 97.992007 96.539371) (end 97.444882 95.992246) (width 0.2) (layer "F.Cu") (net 1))
 (segment (start 110.463463 102.231261) (end 111.881239 102.231261) (width 0.2) (layer "F.Cu") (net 1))
 (segment (start 89.788463 94.231261) (end 89.788463 95.085362) (width 0.2) (layer "F.Cu") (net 1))
 (segment (start 87.913762 92.116277) (end 88.923479 92.116277) (width 0.2) (layer "F.Cu") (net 1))
 (via (at 97.444882 95.992246) (size 0.6) (drill 0.3) (layers "F.Cu" "B.Cu") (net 1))
 (via (at 110.463463 102.231261) (size 0.6) (drill 0.3) (layers "F.Cu" "B.Cu") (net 1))
 (via (at 99.263463 99.731261) (size 0.6) (drill 0.3) (layers "F.Cu" "B.Cu") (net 1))
 (via (at 101.863463 99.831261) (size 0.6) (drill 0.3) (layers "F.Cu" "B.Cu") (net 1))
 (segment (start 99.263463 99.731261) (end 101.763463 99.731261) (width 0.2) (layer "B.Cu") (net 1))
 (segment (start 94.383762 92.931126) (end 97.444882 95.992246) (width 0.2) (layer "B.Cu") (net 1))
 (segment (start 94.383762 90.966277) (end 94.398479 90.966277) (width 0.2) (layer "B.Cu") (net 1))
 (segment (start 101.763463 99.731261) (end 101.863463 99.831261) (width 0.2) (layer "B.Cu") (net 1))
 (segment (start 86.763762 90.966277) (end 85.513463 92.216576) (width 0.2) (layer "B.Cu") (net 1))
 (segment (start 94.383762 90.966277) (end 94.383762 92.931126) (width 0.2) (layer "B.Cu") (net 1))
 (segment (start 108.063463 99.831261) (end 110.463463 102.231261) (width 0.2) (layer "B.Cu") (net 1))
 (segment (start 101.863463 99.831261) (end 108.063463 99.831261) (width 0.2) (layer "B.Cu") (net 1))
 (segment (start 85.513463 92.216576) (end 85.513463 97.621261) (width 0.2) (layer "B.Cu") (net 1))
 (segment (start 86.768405 91.018739) (end 87.918405 89.868739) (width 0.2) (layer "B.Cu") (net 1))
 (segment (start 85.513463 97.621261) (end 86.663463 98.771261) (width 0.2) (layer "B.Cu") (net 1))
 (segment (start 93.238405 89.868739) (end 94.388405 91.018739) (width 0.2) (layer "B.Cu") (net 1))
 (segment (start 87.918405 89.868739) (end 93.238405 89.868739) (width 0.2) (layer "B.Cu") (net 1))
 (segment (start 95.663463 97.506261) (end 97.313463 97.506261) (width 0.2) (layer "F.Cu") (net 30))
 (segment (start 97.313463 97.506261) (end 98.038463 98.231261) (width 0.2) (layer "F.Cu") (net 30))
 (segment (start 92.163463 104.284907) (end 92.151452 104.272896) (width 0.2) (layer "F.Cu") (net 31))
 (segment (start 92.163463 105.177614) (end 92.163463 104.284907) (width 0.2) (layer "F.Cu") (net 31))
 (segment (start 88.663463 96.581261) (end 89.834362 96.581261) (width 0.2) (layer "F.Cu") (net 29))
 (segment (start 89.834362 96.581261) (end 89.963935 96.710834) (width 0.2) (layer "F.Cu") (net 29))
 (segment (start 104.963463 95.506261) (end 104.688463 95.231261) (width 0.2) (layer "F.Cu") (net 26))
 (segment (start 89.243463 109.231261) (end 89.243463 103.891261) (width 0.2) (layer "F.Cu") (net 26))
 (segment (start 92.743463 95.231261) (end 86.663463 101.311261) (width 0.2) (layer "F.Cu") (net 26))
 (segment (start 89.243463 103.891261) (end 86.663463 101.311261) (width 0.2) (layer "F.Cu") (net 26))
 (segment (start 104.963463 95.931261) (end 104.963463 95.506261) (width 0.2) (layer "F.Cu") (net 26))
 (segment (start 104.688463 95.231261) (end 92.743463 95.231261) (width 0.2) (layer "F.Cu") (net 26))
 (segment (start 112.123463 106.731261) (end 108.163463 106.731261) (width 0.2) (layer "F.Cu") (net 20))
 (segment (start 106.563463 105.131261) (end 108.163463 106.731261) (width 0.2) (layer "F.Cu") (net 20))
 (segment (start 114.623463 109.231261) (end 112.123463 106.731261) (width 0.2) (layer "F.Cu") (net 20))
 (segment (start 106.563463 104.531261) (end 106.563463 105.131261) (width 0.2) (layer "F.Cu") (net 20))
 (segment (start 100.363463 97.706261) (end 102.138463 95.931261) (width 0.2) (layer "F.Cu") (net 28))
 (segment (start 100.363463 105.731261) (end 100.363463 97.706261) (width 0.2) (layer "F.Cu") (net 28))
 (segment (start 102.138463 95.931261) (end 103.363463 95.931261) (width 0.2) (layer "F.Cu") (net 28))
 (segment (start 96.863463 109.231261) (end 100.363463 105.731261) (width 0.2) (layer "F.Cu") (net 28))
 (segment (start 103.363463 108.131261) (end 103.363463 104.531261) (width 0.2) (layer "F.Cu") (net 16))
 (segment (start 104.463463 109.231261) (end 103.363463 108.131261) (width 0.2) (layer "F.Cu") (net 16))
 (segment (start 91.877728 96.945526) (end 95.163463 100.231261) (width 0.2) (layer "F.Cu") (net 3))
 (segment (start 105.263463 94.831261) (end 105.763463 95.331261) (width 0.2) (layer "F.Cu") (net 3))
 (segment (start 91.843762 90.966277) (end 95.708746 94.831261) (width 0.2) (layer "F.Cu") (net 3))
 (segment (start 95.163463 100.231261) (end 95.163463 101.231261) (width 0.2) (layer "F.Cu") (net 3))
 (segment (start 95.708746 94.831261) (end 105.263463 94.831261) (width 0.2) (layer "F.Cu") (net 3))
 (segment (start 105.763463 95.331261) (end 105.763463 95.931261) (width 0.2) (layer "F.Cu") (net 3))
 (segment (start 98.063463 99.731261) (end 96.838463 100.956261) (width 0.2) (layer "F.Cu") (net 3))
 (segment (start 96.838463 100.956261) (end 95.663463 100.956261) (width 0.2) (layer "F.Cu") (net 3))
 (via (at 91.877728 96.945526) (size 0.6) (drill 0.3) (layers "F.Cu" "B.Cu") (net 3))
 (via (at 95.163463 101.231261) (size 0.6) (drill 0.3) (layers "F.Cu" "B.Cu") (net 3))
 (segment (start 91.877728 96.945526) (end 91.843762 96.91156) (width 0.2) (layer "B.Cu") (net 3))
 (segment (start 88.943463 106.391261) (end 91.783463 109.231261) (width 0.2) (layer "B.Cu") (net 3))
 (segment (start 90.003463 106.391261) (end 95.163463 101.231261) (width 0.2) (layer "B.Cu") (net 3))
 (segment (start 91.843762 96.91156) (end 91.843762 90.966277) (width 0.2) (layer "B.Cu") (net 3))
 (segment (start 88.943463 106.391261) (end 90.003463 106.391261) (width 0.2) (layer "B.Cu") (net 3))
 (segment (start 86.663463 106.391261) (end 88.943463 106.391261) (width 0.2) (layer "B.Cu") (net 3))
 (via (at 104.163463 95.931261) (size 0.6) (drill 0.3) (layers "F.Cu" "B.Cu") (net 27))
 (segment (start 86.663463 103.851261) (end 85.513463 105.001261) (width 0.2) (layer "B.Cu") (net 27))
 (segment (start 104.163463 95.931261) (end 103.963463 95.931261) (width 0.2) (layer "B.Cu") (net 27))
 (segment (start 93.783463 96.731261) (end 103.163463 96.731261) (width 0.2) (layer "B.Cu") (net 27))
 (segment (start 103.963463 95.931261) (end 103.163463 96.731261) (width 0.2) (layer "B.Cu") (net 27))
 (segment (start 85.513463 105.001261) (end 85.513463 108.041261) (width 0.2) (layer "B.Cu") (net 27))
 (segment (start 85.513463 108.041261) (end 86.703463 109.231261) (width 0.2) (layer "B.Cu") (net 27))
 (segment (start 86.663463 103.851261) (end 93.783463 96.731261) (width 0.2) (layer "B.Cu") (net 27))
 (segment (start 105.763463 104.896947) (end 105.763463 104.531261) (width 0.2) (layer "F.Cu") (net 19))
 (segment (start 112.083463 109.231261) (end 109.983463 107.131261) (width 0.2) (layer "F.Cu") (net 19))
 (segment (start 107.997777 107.131261) (end 105.763463 104.896947) (width 0.2) (layer "F.Cu") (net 19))
 (segment (start 109.983463 107.131261) (end 107.997777 107.131261) (width 0.2) (layer "F.Cu") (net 19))
 (segment (start 111.363463 109.231261) (end 112.083463 109.231261) (width 0.2) (layer "F.Cu") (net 19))
 (segment (start 101.438463 98.231261) (end 101.163463 98.506261) (width 0.2) (layer "F.Cu") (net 13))
 (segment (start 101.163463 98.506261) (end 101.163463 108.471261) (width 0.2) (layer "F.Cu") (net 13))
 (segment (start 101.163463 108.471261) (end 101.923463 109.231261) (width 0.2) (layer "F.Cu") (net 13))
 (segment (start 101.863463 98.231261) (end 101.438463 98.231261) (width 0.2) (layer "F.Cu") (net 13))
 (segment (start 109.543463 109.231261) (end 109.063463 109.231261) (width 0.2) (layer "F.Cu") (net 18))
 (segment (start 109.063463 109.231261) (end 104.963463 105.131261) (width 0.2) (layer "F.Cu") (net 18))
 (segment (start 104.963463 105.131261) (end 104.963463 104.531261) (width 0.2) (layer "F.Cu") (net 18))
 (segment (start 100.763463 97.931261) (end 101.263463 97.431261) (width 0.2) (layer "F.Cu") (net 12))
 (segment (start 101.263463 97.431261) (end 101.863463 97.431261) (width 0.2) (layer "F.Cu") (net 12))
 (segment (start 99.403463 109.231261) (end 100.763463 107.871261) (width 0.2) (layer "F.Cu") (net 12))
 (segment (start 100.763463 107.871261) (end 100.763463 97.931261) (width 0.2) (layer "F.Cu") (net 12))
 (segment (start 104.163463 106.391261) (end 104.163463 104.531261) (width 0.2) (layer "F.Cu") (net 17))
 (segment (start 107.003463 109.231261) (end 104.163463 106.391261) (width 0.2) (layer "F.Cu") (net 17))
 (segment (start 111.264776 105.731261) (end 108.163463 105.731261) (width 0.2) (layer "F.Cu") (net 11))
 (segment (start 107.363463 104.931261) (end 107.363463 104.531261) (width 0.2) (layer "F.Cu") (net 11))
 (segment (start 114.683762 90.966277) (end 114.683762 102.312275) (width 0.2) (layer "F.Cu") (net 11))
 (segment (start 108.163463 105.731261) (end 107.363463 104.931261) (width 0.2) (layer "F.Cu") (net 11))
 (segment (start 114.683762 102.312275) (end 111.264776 105.731261) (width 0.2) (layer "F.Cu") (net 11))
 (segment (start 112.799182 96.701697) (end 112.799182 102.499798) (width 0.2) (layer "F.Cu") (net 8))
 (segment (start 107.063762 90.966277) (end 112.799182 96.701697) (width 0.2) (layer "F.Cu") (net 8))
 (segment (start 112.267719 103.031261) (end 110.463463 103.031261) (width 0.2) (layer "F.Cu") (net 8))
 (segment (start 112.799182 102.499798) (end 112.267719 103.031261) (width 0.2) (layer "F.Cu") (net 8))
 (via (at 92.163463 103.231261) (size 0.6) (drill 0.3) (layers "F.Cu" "B.Cu") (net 8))
 (segment (start 107.063762 95.830962) (end 105.394724 97.5) (width 0.2) (layer "B.Cu") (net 8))
 (segment (start 107.063762 90.966277) (end 107.063762 95.830962) (width 0.2) (layer "B.Cu") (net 8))
 (segment (start 105.394724 97.5) (end 97.894724 97.5) (width 0.2) (layer "B.Cu") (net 8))
 (segment (start 97.894724 97.5) (end 92.163463 103.231261) (width 0.2) (layer "B.Cu") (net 8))
 (segment (start 108.963463 95.331261) (end 108.963463 95.931261) (width 0.2) (layer "F.Cu") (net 5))
 (segment (start 107.663463 94.031261) (end 108.963463 95.331261) (width 0.2) (layer "F.Cu") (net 5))
 (segment (start 102.528746 94.031261) (end 107.663463 94.031261) (width 0.2) (layer "F.Cu") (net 5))
 (segment (start 99.463762 90.966277) (end 102.528746 94.031261) (width 0.2) (layer "F.Cu") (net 5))
 (segment (start 96.923762 90.966277) (end 100.388746 94.431261) (width 0.2) (layer "F.Cu") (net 4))
 (segment (start 100.388746 94.431261) (end 107.263463 94.431261) (width 0.2) (layer "F.Cu") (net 4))
 (segment (start 108.163463 95.331261) (end 108.163463 95.931261) (width 0.2) (layer "F.Cu") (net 4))
 (segment (start 107.263463 94.431261) (end 108.163463 95.331261) (width 0.2) (layer "F.Cu") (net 4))
 (segment (start 111.333405 104.531261) (end 108.963463 104.531261) (width 0.2) (layer "F.Cu") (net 9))
 (segment (start 109.603762 90.966277) (end 113.199182 94.561697) (width 0.2) (layer "F.Cu") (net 9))
 (segment (start 113.199182 94.561697) (end 113.199182 102.665484) (width 0.2) (layer "F.Cu") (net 9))
 (segment (start 113.199182 102.665484) (end 111.333405 104.531261) (width 0.2) (layer "F.Cu") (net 9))
 (segment (start 113.599182 92.421697) (end 112.143762 90.966277) (width 0.2) (layer "F.Cu") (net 10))
 (segment (start 108.163463 104.531261) (end 108.163463 104.956261) (width 0.2) (layer "F.Cu") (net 10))
 (segment (start 108.438463 105.231261) (end 111.199091 105.231261) (width 0.2) (layer "F.Cu") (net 10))
 (segment (start 108.163463 104.956261) (end 108.438463 105.231261) (width 0.2) (layer "F.Cu") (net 10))
 (segment (start 113.599182 102.83117) (end 113.599182 92.421697) (width 0.2) (layer "F.Cu") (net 10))
 (segment (start 111.199091 105.231261) (end 113.599182 102.83117) (width 0.2) (layer "F.Cu") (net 10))
 (segment (start 110.463463 96.265575) (end 110.463463 97.431261) (width 0.2) (layer "F.Cu") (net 6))
 (segment (start 107.829149 93.631261) (end 110.463463 96.265575) (width 0.2) (layer "F.Cu") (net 6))
 (segment (start 104.648746 93.631261) (end 107.829149 93.631261) (width 0.2) (layer "F.Cu") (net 6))
 (segment (start 101.983762 90.966277) (end 104.648746 93.631261) (width 0.2) (layer "F.Cu") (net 6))
 (segment (start 104.523762 90.966277) (end 106.788746 93.231261) (width 0.2) (layer "F.Cu") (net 7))
 (segment (start 111.163463 98.131261) (end 111.063463 98.231261) (width 0.2) (layer "F.Cu") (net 7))
 (segment (start 111.063463 98.231261) (end 110.463463 98.231261) (width 0.2) (layer "F.Cu") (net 7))
 (segment (start 111.163463 96.399889) (end 111.163463 98.131261) (width 0.2) (layer "F.Cu") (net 7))
 (segment (start 107.994835 93.231261) (end 111.163463 96.399889) (width 0.2) (layer "F.Cu") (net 7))
 (segment (start 106.788746 93.231261) (end 107.994835 93.231261) (width 0.2) (layer "F.Cu") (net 7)))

